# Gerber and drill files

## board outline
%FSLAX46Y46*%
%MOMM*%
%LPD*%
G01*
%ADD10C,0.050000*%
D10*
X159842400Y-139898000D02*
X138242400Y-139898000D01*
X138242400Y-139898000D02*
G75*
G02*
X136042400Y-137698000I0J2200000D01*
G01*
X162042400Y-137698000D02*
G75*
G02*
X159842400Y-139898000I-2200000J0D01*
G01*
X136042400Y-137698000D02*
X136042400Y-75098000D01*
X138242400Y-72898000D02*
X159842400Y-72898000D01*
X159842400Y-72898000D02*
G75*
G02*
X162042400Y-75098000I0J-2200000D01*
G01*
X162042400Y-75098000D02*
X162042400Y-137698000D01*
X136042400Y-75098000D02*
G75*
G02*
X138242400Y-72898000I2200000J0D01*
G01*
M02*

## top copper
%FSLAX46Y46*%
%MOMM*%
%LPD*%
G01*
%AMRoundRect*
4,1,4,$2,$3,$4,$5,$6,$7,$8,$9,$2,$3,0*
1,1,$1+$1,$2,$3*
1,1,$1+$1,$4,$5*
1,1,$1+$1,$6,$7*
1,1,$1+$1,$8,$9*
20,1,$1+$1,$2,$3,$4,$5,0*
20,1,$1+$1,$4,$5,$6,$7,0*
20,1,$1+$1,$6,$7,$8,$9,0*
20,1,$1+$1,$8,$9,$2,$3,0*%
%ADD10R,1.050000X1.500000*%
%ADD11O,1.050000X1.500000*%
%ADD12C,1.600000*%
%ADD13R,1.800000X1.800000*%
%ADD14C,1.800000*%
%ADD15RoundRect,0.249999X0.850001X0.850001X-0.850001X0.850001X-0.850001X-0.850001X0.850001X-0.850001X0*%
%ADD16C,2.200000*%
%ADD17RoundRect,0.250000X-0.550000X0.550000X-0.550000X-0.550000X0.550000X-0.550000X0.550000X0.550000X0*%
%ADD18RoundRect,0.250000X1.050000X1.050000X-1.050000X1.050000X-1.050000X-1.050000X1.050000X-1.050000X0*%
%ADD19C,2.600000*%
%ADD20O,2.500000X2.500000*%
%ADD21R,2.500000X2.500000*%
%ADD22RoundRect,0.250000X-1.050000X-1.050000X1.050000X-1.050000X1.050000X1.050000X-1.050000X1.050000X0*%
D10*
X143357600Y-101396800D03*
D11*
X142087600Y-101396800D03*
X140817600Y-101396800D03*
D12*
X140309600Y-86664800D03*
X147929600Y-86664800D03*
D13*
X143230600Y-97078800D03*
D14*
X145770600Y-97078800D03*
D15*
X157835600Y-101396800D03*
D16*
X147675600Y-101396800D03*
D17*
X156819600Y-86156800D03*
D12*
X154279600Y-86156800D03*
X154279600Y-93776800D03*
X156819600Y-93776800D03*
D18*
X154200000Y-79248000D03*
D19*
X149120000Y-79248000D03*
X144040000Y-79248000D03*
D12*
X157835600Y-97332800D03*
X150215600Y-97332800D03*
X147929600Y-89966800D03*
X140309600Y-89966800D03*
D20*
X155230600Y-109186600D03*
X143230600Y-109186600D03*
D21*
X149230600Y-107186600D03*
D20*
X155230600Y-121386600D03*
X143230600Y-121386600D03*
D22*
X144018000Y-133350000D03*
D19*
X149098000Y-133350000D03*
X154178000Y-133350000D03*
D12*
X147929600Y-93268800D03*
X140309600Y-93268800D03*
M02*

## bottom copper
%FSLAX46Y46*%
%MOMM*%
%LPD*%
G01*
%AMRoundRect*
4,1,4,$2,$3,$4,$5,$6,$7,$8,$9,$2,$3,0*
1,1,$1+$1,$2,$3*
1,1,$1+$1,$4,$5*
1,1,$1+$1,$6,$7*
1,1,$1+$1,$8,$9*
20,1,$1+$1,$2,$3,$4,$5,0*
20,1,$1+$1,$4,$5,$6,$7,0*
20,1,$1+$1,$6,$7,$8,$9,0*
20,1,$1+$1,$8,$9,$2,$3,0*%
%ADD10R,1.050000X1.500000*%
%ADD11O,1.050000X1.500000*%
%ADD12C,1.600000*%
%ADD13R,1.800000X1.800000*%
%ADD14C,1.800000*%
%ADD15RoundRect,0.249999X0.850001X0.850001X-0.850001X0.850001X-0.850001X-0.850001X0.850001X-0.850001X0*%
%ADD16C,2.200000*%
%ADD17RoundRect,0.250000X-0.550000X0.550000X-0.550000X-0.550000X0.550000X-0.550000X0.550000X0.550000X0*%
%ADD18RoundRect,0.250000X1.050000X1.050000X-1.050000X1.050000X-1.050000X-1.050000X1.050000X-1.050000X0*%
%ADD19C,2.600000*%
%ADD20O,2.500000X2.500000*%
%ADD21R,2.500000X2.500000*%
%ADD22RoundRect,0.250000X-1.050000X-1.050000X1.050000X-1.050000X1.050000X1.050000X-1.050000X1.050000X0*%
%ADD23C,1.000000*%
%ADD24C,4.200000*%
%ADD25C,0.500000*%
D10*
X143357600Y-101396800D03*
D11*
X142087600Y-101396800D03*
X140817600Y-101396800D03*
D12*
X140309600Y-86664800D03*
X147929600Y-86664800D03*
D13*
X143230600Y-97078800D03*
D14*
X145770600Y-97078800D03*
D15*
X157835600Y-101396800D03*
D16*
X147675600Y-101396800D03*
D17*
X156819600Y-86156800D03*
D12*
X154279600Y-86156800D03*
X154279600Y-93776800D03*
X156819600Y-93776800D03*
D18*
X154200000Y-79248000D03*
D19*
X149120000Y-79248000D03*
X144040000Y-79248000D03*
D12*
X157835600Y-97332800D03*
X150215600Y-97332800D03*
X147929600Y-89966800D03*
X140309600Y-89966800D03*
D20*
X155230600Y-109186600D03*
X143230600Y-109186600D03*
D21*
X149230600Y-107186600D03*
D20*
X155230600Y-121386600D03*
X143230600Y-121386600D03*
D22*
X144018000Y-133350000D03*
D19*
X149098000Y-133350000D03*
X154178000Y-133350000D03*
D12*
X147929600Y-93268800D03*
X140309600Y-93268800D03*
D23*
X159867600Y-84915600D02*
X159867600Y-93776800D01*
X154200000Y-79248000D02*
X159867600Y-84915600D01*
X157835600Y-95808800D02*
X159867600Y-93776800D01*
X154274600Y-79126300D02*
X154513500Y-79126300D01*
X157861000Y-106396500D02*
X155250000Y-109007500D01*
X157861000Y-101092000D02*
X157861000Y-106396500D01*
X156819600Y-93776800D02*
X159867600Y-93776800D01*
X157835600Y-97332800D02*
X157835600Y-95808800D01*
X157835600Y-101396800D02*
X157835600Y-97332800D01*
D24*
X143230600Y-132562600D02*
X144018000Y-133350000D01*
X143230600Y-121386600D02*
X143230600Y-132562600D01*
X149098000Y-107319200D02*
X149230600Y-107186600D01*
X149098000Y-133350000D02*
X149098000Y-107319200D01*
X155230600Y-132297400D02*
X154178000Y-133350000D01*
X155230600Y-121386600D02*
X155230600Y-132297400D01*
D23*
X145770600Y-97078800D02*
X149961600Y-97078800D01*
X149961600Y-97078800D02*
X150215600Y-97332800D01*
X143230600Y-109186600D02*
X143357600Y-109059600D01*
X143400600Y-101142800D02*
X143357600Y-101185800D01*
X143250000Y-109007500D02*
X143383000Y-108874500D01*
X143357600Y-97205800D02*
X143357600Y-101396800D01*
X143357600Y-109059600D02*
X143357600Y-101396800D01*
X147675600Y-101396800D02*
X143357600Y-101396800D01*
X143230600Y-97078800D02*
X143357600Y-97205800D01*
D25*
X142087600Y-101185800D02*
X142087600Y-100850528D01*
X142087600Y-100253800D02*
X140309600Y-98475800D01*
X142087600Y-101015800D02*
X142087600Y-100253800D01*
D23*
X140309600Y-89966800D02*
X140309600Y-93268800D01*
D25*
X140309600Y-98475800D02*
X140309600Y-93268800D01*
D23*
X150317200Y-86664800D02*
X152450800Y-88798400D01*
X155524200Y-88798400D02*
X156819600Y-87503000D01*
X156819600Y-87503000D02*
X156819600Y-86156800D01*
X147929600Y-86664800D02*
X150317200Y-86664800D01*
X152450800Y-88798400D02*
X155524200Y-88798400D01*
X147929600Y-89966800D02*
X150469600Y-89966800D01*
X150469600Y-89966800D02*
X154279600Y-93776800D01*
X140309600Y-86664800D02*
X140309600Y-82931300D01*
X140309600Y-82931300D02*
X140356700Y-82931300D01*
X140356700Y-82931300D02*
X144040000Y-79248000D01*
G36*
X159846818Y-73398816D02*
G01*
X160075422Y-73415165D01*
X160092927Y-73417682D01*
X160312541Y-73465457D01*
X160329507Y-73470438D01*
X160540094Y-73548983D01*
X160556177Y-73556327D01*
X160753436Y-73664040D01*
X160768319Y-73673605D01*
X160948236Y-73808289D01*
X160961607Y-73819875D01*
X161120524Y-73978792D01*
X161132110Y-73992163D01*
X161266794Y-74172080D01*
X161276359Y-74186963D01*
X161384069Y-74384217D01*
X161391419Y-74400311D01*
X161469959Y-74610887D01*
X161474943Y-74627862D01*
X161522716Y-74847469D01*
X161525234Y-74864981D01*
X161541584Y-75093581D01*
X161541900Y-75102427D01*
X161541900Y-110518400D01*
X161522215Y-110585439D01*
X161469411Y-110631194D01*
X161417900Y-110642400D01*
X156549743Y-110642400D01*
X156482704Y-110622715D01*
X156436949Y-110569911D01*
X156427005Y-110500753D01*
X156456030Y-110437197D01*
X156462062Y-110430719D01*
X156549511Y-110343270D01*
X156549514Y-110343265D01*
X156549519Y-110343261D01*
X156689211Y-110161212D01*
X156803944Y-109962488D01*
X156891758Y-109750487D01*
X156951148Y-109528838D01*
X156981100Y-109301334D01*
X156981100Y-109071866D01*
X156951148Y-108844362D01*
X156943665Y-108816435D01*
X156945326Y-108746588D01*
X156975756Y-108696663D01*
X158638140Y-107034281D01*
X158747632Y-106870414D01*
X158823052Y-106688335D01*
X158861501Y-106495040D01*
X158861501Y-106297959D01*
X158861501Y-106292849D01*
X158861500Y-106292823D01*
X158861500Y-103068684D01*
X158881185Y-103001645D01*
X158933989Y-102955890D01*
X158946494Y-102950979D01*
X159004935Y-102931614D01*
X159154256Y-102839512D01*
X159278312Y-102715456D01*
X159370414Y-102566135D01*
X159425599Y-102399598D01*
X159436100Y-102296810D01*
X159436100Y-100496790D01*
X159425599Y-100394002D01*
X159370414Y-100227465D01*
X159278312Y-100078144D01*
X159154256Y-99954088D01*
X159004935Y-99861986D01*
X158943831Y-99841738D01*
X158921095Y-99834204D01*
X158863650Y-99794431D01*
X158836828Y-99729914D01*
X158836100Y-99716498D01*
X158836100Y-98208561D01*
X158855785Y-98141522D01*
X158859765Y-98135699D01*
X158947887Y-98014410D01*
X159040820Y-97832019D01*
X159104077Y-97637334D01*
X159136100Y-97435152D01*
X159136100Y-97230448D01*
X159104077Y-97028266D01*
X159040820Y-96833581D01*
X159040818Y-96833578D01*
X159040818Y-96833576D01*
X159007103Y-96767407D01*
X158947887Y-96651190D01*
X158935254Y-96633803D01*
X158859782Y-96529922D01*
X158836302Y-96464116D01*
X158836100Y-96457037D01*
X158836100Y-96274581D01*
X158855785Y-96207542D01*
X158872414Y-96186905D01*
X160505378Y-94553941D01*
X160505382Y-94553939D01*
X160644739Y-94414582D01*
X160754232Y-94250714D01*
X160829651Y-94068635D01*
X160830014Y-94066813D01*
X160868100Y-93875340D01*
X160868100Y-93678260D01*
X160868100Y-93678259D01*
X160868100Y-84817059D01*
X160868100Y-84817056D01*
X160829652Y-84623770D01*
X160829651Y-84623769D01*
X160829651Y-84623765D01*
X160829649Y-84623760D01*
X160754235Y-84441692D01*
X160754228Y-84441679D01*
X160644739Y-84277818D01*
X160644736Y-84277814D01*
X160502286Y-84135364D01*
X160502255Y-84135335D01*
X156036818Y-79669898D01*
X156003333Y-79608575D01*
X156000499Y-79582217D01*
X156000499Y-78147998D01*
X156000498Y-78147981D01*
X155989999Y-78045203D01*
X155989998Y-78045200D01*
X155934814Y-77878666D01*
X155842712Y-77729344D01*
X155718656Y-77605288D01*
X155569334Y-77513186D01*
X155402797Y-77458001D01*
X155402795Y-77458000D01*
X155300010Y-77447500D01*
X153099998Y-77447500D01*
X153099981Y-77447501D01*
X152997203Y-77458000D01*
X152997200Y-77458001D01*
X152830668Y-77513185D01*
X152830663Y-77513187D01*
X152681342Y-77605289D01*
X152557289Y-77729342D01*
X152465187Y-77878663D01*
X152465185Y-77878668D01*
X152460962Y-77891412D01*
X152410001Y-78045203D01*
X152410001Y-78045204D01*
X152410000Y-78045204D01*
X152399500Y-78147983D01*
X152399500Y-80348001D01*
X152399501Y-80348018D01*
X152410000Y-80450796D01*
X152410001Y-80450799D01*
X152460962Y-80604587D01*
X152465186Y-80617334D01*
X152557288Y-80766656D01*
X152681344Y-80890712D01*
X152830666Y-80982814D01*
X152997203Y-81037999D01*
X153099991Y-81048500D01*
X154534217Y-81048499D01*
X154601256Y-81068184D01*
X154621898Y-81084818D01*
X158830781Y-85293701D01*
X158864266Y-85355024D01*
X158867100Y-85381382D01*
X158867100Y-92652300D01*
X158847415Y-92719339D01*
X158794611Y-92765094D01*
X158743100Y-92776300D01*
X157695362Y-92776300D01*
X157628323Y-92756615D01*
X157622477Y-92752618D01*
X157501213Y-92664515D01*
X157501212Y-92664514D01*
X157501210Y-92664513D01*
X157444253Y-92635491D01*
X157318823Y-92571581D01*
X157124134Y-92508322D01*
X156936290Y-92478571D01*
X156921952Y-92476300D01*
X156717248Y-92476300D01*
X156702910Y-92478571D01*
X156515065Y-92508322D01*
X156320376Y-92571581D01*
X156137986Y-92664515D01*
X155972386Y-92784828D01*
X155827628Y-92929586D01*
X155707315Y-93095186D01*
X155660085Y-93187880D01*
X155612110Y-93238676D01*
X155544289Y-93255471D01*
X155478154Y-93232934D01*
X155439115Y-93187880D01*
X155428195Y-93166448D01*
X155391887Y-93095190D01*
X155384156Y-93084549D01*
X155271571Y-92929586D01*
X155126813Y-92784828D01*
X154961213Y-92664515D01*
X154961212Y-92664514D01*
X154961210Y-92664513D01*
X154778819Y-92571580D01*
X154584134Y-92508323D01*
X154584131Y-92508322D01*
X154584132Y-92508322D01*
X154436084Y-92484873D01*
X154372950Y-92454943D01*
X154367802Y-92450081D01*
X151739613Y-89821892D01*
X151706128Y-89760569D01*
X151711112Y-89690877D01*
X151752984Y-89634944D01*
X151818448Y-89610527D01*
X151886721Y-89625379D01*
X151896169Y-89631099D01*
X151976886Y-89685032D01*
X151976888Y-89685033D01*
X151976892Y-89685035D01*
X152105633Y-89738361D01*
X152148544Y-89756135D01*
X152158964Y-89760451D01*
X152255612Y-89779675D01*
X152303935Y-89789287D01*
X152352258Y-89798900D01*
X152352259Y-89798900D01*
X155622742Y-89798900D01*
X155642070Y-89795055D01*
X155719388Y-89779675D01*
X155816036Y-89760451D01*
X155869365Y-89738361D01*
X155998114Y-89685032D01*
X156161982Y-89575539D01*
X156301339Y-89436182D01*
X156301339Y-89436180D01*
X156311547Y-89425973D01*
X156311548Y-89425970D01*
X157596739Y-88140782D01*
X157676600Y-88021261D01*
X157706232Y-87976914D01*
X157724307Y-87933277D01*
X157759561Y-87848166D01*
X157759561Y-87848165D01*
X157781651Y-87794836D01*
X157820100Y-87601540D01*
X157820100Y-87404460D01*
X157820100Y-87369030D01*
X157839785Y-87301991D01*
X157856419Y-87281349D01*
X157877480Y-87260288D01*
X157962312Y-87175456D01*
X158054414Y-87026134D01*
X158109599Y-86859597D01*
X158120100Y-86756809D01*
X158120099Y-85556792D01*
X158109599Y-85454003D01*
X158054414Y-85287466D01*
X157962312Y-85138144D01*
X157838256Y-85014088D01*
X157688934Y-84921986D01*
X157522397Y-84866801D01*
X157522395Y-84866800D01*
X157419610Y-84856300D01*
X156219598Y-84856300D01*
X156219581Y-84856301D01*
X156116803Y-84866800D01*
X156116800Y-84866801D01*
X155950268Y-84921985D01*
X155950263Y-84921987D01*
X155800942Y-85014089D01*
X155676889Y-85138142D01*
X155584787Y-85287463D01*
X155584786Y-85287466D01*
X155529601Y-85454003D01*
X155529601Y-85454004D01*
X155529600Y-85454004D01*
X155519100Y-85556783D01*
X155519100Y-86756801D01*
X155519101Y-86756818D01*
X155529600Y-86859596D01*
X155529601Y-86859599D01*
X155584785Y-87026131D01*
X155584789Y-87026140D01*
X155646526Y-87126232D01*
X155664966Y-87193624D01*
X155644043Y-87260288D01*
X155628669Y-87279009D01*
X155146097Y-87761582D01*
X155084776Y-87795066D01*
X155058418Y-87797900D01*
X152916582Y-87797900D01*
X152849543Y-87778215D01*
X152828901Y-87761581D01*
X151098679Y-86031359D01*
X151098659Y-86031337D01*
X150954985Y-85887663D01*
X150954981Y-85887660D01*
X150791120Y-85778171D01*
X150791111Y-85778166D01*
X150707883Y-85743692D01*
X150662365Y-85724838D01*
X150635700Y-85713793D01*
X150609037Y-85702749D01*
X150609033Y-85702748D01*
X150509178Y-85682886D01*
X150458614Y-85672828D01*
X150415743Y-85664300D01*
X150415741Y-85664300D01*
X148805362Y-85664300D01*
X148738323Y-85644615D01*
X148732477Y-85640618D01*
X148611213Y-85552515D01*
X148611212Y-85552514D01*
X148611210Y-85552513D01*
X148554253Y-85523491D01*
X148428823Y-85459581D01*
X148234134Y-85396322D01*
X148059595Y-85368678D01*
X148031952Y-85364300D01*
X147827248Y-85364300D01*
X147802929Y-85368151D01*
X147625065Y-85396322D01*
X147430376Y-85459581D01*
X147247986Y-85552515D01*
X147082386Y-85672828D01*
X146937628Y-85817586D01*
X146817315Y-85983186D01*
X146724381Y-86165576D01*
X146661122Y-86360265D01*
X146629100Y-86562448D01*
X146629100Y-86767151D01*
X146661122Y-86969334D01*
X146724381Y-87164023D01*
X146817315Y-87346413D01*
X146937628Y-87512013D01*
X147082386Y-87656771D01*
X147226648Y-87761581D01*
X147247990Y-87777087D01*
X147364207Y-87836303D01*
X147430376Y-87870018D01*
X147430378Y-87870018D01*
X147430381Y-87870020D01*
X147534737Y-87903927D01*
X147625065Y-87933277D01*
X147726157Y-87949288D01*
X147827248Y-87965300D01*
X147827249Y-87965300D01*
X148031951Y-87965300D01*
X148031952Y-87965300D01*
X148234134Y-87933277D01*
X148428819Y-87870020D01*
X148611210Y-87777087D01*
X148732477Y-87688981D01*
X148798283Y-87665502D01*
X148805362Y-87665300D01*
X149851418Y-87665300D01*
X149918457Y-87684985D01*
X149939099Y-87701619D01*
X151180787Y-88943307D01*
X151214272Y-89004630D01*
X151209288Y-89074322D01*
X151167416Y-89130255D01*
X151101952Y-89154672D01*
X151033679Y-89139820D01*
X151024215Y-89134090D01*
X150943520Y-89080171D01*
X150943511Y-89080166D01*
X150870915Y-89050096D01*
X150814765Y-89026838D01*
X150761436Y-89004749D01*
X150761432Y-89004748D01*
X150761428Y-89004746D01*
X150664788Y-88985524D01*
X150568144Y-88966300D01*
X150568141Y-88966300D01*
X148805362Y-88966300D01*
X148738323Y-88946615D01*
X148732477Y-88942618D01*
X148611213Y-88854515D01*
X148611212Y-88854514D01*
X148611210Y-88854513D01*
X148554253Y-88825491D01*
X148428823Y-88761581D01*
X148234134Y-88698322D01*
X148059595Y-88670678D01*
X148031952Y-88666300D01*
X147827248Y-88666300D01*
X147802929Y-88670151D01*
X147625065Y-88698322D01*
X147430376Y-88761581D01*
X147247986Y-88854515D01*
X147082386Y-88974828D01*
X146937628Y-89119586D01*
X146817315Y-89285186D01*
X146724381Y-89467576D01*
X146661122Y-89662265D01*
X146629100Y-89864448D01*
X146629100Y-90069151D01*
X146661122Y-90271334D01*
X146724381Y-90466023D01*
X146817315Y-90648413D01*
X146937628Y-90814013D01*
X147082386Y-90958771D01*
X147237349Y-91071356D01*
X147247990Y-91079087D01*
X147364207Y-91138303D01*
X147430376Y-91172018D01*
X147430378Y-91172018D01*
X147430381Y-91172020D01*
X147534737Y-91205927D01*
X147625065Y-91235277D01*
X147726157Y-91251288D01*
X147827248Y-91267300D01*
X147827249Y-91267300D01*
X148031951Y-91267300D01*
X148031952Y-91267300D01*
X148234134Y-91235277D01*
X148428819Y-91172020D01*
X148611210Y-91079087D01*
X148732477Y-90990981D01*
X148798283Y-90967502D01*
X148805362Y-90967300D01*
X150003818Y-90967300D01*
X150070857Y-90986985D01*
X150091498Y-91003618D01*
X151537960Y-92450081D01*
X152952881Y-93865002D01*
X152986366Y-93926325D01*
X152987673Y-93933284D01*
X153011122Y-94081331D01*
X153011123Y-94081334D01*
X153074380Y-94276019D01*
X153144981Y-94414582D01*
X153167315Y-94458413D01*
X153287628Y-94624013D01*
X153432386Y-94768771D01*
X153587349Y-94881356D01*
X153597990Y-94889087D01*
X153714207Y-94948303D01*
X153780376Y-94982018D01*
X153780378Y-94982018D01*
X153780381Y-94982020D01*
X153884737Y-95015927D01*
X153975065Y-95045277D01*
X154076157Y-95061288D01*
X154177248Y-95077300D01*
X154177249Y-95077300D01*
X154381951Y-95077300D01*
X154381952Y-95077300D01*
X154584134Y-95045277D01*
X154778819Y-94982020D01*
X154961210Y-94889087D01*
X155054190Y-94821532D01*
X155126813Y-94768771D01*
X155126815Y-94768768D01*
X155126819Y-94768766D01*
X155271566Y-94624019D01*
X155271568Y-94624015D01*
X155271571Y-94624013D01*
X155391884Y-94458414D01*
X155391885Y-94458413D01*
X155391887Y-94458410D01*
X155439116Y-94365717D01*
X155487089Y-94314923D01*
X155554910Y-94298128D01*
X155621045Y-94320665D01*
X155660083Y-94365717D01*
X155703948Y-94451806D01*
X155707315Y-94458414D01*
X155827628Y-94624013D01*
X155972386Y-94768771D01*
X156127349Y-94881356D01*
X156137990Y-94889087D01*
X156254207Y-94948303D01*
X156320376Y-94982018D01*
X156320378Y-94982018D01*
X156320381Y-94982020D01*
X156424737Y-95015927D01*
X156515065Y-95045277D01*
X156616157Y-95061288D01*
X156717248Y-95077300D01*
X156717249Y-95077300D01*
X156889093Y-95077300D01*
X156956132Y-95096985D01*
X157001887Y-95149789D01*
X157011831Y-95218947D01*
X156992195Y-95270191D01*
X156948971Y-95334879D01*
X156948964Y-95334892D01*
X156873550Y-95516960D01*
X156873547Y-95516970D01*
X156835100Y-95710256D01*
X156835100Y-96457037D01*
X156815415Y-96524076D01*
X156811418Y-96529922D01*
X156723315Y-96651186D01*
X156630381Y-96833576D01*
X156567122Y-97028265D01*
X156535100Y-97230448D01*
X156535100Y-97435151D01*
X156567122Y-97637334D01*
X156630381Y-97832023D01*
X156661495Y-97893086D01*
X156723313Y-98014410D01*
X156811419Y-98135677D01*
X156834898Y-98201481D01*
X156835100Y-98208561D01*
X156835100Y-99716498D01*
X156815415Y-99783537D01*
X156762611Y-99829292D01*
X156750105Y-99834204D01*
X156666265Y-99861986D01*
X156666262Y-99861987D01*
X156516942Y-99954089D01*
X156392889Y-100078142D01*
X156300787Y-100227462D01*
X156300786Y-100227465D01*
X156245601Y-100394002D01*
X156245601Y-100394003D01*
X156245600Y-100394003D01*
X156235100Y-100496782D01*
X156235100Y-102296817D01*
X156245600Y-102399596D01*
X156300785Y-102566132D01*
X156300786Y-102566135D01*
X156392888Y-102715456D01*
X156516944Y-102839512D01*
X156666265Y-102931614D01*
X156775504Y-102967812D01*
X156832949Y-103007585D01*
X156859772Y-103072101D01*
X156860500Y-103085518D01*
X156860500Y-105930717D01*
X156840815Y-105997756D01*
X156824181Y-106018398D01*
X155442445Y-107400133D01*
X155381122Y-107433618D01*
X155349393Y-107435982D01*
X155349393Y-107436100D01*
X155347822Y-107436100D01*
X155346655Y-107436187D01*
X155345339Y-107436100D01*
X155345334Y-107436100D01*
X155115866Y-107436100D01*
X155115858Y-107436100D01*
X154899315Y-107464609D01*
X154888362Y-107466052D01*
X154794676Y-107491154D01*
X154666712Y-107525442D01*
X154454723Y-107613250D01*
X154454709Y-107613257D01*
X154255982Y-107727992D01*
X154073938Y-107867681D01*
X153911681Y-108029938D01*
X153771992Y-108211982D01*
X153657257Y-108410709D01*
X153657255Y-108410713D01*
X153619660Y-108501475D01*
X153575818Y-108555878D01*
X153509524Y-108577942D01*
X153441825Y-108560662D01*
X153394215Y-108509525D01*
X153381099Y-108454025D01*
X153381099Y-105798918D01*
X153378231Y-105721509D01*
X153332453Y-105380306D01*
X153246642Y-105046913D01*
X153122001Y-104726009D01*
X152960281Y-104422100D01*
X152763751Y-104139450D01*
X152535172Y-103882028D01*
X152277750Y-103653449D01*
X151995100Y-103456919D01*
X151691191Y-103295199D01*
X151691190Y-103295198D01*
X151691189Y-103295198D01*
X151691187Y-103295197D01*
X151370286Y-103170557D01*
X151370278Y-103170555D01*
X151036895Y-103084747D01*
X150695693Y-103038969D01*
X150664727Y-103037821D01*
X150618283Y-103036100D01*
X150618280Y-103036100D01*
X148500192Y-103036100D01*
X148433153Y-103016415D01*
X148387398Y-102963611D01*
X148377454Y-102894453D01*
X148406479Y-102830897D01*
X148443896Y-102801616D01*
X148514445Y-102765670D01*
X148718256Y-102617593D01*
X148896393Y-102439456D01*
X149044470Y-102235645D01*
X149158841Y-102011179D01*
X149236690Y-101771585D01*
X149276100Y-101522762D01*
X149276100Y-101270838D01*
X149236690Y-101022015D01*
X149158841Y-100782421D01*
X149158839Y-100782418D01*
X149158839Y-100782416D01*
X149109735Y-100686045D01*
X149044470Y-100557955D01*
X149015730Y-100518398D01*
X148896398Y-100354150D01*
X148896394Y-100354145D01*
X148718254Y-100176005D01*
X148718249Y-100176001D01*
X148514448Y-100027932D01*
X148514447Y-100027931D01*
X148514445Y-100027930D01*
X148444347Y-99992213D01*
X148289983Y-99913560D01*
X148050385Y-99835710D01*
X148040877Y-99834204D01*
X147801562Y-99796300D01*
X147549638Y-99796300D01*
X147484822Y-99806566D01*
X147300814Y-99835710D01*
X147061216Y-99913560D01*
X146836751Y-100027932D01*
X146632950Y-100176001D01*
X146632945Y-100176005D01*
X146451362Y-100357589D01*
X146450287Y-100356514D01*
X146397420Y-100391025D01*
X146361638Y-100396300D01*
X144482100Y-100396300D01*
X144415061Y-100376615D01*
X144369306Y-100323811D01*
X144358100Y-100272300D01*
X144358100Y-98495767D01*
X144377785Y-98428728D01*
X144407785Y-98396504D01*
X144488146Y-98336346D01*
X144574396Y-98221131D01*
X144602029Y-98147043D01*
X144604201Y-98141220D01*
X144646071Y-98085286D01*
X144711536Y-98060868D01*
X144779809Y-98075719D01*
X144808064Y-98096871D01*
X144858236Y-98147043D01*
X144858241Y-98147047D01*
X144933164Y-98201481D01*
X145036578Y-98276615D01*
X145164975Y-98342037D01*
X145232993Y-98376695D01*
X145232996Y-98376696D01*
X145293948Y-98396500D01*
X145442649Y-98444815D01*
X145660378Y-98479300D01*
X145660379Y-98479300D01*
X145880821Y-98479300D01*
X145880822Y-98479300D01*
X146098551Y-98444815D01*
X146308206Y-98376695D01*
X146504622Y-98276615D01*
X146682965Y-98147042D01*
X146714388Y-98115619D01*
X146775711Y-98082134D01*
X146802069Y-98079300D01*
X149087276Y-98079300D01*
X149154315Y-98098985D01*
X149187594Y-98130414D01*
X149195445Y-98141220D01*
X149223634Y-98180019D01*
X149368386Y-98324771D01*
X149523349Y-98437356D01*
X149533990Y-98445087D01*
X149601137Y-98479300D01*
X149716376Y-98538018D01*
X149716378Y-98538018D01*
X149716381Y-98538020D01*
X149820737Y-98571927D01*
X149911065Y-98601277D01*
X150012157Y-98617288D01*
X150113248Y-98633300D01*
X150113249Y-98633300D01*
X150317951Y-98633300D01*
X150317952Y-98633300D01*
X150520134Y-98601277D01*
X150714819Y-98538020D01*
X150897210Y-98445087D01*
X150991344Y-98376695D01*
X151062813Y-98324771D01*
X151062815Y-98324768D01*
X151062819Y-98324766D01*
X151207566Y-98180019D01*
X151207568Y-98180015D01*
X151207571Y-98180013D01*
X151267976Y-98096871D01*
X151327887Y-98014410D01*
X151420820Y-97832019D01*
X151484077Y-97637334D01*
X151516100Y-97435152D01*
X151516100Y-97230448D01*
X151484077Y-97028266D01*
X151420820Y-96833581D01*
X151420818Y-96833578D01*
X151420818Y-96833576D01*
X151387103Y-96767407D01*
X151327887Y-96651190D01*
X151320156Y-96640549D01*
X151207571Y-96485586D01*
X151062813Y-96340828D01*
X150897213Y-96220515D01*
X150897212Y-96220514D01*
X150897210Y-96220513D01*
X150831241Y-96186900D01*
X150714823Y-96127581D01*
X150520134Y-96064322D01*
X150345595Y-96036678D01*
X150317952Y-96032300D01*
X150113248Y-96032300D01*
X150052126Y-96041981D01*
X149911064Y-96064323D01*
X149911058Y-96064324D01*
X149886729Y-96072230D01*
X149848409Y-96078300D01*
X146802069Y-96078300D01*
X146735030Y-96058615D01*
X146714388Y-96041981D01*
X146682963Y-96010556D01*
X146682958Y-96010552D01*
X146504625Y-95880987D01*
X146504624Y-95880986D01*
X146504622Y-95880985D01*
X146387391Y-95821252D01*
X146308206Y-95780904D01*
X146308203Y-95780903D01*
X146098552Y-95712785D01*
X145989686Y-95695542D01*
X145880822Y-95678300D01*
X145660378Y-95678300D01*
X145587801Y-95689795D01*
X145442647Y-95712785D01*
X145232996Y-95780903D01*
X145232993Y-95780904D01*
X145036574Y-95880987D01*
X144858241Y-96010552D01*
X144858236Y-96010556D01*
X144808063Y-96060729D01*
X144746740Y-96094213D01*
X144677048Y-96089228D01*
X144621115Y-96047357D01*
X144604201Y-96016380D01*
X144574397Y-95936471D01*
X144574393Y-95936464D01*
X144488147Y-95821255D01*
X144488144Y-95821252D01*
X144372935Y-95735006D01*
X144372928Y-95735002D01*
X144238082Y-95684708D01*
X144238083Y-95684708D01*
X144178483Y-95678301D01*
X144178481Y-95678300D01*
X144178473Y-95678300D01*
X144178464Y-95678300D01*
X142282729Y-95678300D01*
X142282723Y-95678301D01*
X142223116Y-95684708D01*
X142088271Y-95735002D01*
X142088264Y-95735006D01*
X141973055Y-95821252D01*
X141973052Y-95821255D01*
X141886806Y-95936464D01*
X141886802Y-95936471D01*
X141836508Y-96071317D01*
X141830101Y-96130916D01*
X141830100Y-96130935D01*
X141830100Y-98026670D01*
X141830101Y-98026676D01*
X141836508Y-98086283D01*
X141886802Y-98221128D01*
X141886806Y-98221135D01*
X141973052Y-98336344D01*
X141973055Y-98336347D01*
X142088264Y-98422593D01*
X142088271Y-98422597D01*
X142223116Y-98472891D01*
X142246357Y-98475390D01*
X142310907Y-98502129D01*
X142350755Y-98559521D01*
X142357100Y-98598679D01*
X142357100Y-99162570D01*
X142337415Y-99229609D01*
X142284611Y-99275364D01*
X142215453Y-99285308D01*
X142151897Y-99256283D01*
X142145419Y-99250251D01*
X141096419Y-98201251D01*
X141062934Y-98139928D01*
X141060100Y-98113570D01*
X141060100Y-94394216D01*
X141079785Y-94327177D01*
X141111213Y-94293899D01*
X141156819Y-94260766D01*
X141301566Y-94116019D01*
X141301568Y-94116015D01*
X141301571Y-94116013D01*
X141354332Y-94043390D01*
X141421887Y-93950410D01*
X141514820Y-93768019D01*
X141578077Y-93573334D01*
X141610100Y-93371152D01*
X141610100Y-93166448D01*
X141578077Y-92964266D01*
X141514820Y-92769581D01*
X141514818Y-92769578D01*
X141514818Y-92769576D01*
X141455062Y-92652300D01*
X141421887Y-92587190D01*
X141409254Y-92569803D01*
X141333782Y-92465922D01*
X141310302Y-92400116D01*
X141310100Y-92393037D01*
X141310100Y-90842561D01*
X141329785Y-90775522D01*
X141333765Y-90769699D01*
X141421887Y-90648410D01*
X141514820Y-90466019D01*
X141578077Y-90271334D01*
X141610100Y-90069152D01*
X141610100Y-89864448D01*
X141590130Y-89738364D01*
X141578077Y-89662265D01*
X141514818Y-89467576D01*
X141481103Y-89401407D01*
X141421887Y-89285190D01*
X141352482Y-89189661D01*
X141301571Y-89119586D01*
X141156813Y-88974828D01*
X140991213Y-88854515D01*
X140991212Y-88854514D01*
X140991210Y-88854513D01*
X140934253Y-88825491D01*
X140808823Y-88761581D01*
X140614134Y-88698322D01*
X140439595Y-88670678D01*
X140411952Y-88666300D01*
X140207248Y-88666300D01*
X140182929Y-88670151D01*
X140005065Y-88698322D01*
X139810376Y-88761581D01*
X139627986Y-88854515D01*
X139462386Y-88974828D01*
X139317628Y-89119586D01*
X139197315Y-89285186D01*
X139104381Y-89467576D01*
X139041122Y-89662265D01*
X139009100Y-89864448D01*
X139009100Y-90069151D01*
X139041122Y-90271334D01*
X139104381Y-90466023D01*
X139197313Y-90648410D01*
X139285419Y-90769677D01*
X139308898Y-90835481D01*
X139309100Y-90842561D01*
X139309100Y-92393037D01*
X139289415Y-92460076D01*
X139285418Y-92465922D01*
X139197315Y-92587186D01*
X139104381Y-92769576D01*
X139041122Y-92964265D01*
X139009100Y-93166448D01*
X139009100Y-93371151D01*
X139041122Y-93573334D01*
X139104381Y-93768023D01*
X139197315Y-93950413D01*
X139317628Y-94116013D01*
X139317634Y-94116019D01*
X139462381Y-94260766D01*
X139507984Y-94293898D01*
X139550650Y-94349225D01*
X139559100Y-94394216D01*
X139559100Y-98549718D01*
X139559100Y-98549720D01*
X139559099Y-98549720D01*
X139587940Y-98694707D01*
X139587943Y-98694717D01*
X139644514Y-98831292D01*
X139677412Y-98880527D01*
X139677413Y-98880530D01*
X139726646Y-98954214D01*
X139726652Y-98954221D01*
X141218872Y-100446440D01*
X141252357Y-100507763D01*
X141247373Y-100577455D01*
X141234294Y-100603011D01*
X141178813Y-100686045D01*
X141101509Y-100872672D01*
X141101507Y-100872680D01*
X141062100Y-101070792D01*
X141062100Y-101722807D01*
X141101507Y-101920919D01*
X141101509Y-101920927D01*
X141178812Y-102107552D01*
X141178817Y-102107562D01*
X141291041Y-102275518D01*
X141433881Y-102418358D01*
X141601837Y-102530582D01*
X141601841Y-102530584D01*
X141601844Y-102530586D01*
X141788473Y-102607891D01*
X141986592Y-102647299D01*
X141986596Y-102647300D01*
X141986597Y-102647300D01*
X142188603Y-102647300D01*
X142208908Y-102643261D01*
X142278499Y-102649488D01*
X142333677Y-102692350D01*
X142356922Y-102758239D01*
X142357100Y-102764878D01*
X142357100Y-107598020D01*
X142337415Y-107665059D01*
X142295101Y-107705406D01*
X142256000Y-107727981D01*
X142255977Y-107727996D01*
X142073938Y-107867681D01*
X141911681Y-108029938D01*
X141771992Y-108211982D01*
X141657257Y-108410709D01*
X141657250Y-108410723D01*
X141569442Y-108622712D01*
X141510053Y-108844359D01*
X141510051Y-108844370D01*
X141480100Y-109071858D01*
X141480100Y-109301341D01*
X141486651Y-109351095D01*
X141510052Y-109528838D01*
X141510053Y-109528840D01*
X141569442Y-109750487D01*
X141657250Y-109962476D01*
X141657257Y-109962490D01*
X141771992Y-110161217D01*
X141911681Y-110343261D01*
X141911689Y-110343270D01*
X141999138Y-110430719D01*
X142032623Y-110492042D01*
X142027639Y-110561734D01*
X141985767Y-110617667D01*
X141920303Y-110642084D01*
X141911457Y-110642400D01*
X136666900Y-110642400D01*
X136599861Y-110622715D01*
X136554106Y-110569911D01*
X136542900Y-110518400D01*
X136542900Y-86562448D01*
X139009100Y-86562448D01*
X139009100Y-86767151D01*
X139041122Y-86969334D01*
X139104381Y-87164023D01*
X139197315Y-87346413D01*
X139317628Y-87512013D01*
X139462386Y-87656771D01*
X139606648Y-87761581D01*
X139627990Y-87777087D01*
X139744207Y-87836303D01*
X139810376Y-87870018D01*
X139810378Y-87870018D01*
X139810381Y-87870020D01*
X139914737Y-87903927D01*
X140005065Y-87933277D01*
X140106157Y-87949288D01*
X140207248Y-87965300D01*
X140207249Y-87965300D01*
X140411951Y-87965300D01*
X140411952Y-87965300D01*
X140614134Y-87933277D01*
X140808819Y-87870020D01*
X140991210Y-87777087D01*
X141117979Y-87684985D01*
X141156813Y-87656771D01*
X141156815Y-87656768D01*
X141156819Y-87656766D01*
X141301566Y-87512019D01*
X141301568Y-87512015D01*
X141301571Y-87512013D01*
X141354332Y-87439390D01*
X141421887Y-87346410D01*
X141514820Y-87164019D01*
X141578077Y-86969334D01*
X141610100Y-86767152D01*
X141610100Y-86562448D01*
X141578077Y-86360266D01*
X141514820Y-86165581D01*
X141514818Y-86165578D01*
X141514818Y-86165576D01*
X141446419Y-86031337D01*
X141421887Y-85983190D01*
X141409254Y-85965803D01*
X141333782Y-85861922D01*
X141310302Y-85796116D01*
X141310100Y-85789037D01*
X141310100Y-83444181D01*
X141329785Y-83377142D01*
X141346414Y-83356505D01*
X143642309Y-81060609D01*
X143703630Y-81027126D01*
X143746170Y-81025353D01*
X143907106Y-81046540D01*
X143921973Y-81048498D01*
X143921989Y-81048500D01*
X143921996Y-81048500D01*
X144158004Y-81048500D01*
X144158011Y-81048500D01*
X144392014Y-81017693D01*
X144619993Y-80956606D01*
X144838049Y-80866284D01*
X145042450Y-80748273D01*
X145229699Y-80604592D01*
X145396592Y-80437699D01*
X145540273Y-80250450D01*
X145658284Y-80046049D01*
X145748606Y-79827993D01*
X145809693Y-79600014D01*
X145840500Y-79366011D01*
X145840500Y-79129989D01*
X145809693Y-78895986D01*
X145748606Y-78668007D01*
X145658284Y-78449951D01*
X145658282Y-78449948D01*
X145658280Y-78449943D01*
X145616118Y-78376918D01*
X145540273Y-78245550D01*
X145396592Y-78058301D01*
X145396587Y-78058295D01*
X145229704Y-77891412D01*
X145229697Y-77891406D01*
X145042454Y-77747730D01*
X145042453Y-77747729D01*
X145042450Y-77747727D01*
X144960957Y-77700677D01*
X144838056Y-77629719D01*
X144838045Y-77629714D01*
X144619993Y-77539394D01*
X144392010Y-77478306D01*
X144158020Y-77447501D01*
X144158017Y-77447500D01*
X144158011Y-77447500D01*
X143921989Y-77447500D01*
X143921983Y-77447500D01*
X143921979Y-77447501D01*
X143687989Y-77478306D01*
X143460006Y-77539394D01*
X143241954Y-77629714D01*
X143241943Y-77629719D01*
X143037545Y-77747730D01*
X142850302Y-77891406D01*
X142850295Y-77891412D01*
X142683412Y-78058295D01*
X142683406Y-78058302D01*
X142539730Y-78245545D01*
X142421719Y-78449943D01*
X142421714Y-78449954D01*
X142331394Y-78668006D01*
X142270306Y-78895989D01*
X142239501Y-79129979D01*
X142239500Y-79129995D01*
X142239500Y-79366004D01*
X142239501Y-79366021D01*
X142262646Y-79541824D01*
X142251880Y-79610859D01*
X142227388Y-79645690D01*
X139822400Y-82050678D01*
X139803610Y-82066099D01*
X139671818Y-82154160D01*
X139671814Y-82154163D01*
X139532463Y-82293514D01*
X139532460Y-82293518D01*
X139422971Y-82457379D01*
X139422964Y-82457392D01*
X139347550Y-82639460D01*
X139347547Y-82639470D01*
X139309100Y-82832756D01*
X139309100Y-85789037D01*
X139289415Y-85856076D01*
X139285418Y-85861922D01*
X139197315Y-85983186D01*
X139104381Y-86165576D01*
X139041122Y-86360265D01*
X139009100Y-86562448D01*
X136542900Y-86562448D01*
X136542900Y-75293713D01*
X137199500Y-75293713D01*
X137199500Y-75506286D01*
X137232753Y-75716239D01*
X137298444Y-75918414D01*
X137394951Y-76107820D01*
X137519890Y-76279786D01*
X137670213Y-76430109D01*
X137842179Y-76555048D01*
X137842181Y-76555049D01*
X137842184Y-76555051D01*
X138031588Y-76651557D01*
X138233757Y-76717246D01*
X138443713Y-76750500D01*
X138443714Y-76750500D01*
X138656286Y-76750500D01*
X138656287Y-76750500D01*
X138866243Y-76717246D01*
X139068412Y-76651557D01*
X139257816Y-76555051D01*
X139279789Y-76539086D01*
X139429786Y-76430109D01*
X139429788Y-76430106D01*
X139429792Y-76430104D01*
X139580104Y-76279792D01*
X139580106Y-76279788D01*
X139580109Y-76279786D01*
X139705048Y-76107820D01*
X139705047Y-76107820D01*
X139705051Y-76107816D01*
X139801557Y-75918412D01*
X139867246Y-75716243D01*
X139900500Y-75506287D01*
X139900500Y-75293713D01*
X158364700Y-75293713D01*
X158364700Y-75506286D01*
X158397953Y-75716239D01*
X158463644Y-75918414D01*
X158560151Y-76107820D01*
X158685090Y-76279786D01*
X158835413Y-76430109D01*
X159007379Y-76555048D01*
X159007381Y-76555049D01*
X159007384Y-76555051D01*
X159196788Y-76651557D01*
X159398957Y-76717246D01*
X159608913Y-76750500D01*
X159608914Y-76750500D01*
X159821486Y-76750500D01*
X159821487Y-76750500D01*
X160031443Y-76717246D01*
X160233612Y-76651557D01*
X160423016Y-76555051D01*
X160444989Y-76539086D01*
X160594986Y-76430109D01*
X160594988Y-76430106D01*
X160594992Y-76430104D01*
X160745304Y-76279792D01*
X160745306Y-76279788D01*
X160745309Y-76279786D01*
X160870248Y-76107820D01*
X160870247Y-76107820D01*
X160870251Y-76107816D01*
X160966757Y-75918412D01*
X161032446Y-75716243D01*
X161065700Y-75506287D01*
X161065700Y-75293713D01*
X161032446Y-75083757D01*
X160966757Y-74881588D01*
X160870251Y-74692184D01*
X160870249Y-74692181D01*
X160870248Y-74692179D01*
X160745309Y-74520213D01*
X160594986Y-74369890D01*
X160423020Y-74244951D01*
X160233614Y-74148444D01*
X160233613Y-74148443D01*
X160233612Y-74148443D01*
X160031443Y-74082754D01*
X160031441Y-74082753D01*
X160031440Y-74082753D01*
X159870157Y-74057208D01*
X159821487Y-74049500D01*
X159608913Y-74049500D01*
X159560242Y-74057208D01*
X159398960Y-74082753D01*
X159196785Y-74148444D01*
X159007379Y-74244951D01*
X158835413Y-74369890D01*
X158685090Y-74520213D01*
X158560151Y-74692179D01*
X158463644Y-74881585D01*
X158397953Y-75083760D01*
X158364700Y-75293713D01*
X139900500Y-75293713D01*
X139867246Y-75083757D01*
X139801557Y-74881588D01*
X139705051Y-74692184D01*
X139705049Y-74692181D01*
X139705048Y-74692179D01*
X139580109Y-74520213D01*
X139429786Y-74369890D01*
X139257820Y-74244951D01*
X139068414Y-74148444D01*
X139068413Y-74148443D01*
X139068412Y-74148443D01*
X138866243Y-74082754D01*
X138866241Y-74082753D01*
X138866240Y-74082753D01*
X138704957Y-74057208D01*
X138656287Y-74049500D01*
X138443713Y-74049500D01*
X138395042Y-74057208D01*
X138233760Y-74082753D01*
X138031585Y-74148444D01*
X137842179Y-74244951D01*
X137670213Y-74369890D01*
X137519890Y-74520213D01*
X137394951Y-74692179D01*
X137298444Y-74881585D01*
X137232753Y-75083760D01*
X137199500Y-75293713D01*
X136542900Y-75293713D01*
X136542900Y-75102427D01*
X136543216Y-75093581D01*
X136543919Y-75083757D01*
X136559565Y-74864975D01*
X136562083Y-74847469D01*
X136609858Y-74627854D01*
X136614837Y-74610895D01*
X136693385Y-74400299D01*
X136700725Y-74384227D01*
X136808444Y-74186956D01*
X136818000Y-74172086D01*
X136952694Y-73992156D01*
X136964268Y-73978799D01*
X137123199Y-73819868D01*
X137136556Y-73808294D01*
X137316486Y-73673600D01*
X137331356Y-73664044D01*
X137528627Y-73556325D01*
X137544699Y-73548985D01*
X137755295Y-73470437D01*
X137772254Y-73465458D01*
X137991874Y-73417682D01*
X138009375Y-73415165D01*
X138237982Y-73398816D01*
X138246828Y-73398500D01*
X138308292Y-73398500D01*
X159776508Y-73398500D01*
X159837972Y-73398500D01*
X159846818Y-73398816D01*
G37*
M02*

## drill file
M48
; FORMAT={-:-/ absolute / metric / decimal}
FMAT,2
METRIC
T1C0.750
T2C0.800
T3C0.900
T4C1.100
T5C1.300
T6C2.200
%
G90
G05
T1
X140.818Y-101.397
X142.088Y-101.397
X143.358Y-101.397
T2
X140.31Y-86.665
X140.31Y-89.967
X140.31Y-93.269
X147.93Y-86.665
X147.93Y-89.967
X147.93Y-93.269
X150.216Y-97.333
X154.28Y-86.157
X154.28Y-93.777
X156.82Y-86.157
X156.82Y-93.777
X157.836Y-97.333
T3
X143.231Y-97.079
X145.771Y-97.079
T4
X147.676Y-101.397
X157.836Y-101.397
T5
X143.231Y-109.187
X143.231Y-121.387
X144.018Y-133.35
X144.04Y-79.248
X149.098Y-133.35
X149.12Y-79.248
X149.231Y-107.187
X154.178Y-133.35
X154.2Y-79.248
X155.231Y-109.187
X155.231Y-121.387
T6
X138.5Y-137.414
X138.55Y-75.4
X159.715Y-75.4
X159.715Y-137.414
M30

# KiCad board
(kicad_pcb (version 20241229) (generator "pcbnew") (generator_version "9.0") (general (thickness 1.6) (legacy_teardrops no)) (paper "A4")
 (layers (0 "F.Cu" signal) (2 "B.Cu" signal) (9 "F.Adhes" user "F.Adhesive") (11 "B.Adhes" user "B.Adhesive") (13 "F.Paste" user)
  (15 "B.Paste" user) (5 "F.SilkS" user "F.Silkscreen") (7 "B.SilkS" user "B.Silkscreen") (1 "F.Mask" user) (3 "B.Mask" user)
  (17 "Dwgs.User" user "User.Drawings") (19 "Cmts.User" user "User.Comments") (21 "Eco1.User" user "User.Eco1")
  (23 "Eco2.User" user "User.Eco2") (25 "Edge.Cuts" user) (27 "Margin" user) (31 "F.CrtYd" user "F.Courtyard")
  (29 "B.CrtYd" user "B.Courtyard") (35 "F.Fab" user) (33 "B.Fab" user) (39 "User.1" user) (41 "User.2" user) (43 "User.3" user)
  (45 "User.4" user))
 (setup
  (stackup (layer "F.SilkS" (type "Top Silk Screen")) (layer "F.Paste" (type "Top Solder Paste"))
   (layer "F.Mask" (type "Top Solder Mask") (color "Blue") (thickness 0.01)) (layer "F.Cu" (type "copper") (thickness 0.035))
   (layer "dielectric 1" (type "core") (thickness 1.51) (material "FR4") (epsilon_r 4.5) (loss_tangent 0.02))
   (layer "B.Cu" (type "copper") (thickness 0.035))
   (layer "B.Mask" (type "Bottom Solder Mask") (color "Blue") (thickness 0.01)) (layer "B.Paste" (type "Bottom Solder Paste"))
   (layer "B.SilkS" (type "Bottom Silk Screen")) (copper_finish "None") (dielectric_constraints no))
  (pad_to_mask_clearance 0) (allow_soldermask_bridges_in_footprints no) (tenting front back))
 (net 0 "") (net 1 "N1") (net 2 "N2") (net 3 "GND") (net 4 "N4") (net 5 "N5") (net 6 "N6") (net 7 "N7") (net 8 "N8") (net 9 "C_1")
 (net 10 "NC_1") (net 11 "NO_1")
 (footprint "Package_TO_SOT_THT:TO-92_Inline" (layer "F.Cu") (at 143.3576 101.3968 180)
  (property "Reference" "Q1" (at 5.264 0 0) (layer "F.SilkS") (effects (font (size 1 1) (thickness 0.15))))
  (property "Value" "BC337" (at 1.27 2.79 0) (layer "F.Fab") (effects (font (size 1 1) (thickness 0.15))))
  (pad "1" thru_hole rect (at 0 0 180) (size 1.05 1.5) (drill 0.75) (layers "*.Cu" "*.Mask") (remove_unused_layers no) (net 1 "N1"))
  (pad "2" thru_hole oval (at 1.27 0 180) (size 1.05 1.5) (drill 0.75) (layers "*.Cu" "*.Mask") (remove_unused_layers no) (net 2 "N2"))
  (pad "3" thru_hole oval (at 2.54 0 180) (size 1.05 1.5) (drill 0.75) (layers "*.Cu" "*.Mask") (remove_unused_layers no) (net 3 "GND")))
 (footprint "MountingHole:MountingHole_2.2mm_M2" (layer "F.Cu") (at 159.7152 137.414)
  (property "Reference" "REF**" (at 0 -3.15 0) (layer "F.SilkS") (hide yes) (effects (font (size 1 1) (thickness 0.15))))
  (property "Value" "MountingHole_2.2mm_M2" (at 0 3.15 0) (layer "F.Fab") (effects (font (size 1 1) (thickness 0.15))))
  (pad "" np_thru_hole circle (at 0 0) (size 2.2 2.2) (drill 2.2) (layers "*.Cu" "*.Mask")))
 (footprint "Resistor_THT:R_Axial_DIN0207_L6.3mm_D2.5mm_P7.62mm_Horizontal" (layer "F.Cu") (at 140.3096 86.6648)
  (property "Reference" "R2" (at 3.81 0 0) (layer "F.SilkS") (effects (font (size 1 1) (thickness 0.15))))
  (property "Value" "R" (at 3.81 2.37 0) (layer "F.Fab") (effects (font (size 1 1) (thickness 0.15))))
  (pad "1" thru_hole circle (at 0 0) (size 1.6 1.6) (drill 0.8) (layers "*.Cu" "*.Mask") (remove_unused_layers no) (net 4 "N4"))
  (pad "2" thru_hole circle (at 7.62 0) (size 1.6 1.6) (drill 0.8) (layers "*.Cu" "*.Mask") (remove_unused_layers no) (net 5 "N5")))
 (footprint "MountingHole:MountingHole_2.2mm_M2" (layer "F.Cu") (at 159.7152 75.4)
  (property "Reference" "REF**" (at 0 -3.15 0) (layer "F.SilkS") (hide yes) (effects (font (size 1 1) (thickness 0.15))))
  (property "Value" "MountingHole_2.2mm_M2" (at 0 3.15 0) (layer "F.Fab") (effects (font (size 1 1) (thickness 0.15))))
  (pad "" np_thru_hole circle (at 0 0) (size 2.2 2.2) (drill 2.2) (layers "*.Cu" "*.Mask")))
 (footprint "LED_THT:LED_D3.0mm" (layer "F.Cu") (at 143.2306 97.0788)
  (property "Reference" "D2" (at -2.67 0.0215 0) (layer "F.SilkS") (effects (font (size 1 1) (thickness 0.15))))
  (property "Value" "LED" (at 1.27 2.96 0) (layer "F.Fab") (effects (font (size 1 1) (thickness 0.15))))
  (pad "1" thru_hole rect (at 0 0) (size 1.8 1.8) (drill 0.9) (layers "*.Cu" "*.Mask") (remove_unused_layers no) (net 1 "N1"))
  (pad "2" thru_hole circle (at 2.54 0) (size 1.8 1.8) (drill 0.9) (layers "*.Cu" "*.Mask") (remove_unused_layers no) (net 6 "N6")))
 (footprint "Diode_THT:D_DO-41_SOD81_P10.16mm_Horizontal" (layer "F.Cu") (at 157.8356 101.3968 180)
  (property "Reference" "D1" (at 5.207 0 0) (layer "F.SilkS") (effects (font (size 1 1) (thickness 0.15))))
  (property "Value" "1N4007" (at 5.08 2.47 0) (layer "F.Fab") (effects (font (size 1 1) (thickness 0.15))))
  (pad "1" thru_hole roundrect (at 0 0 180) (size 2.2 2.2) (drill 1.1) (layers "*.Cu" "*.Mask") (remove_unused_layers no)
   (roundrect_rratio 0.113636) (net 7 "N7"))
  (pad "2" thru_hole circle (at 10.16 0 180) (size 2.2 2.2) (drill 1.1) (layers "*.Cu" "*.Mask") (remove_unused_layers no) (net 1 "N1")))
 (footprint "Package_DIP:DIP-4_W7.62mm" (layer "F.Cu") (at 156.8196 86.1568 -90)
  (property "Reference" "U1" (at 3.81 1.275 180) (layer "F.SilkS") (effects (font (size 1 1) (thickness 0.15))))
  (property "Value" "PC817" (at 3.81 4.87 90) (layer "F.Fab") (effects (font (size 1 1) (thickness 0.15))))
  (pad "1" thru_hole roundrect (at 0 0 270) (size 1.6 1.6) (drill 0.8) (layers "*.Cu" "*.Mask") (remove_unused_layers no)
   (roundrect_rratio 0.15625) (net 5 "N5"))
  (pad "2" thru_hole circle (at 0 2.54 270) (size 1.6 1.6) (drill 0.8) (layers "*.Cu" "*.Mask") (remove_unused_layers no) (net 3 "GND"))
  (pad "3" thru_hole circle (at 7.62 2.54 270) (size 1.6 1.6) (drill 0.8) (layers "*.Cu" "*.Mask") (remove_unused_layers no) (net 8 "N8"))
  (pad "4" thru_hole circle (at 7.62 0 270) (size 1.6 1.6) (drill 0.8) (layers "*.Cu" "*.Mask") (remove_unused_layers no) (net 7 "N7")))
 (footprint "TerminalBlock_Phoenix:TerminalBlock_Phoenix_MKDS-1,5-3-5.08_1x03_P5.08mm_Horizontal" (layer "F.Cu") (at 154.2 79.248 180)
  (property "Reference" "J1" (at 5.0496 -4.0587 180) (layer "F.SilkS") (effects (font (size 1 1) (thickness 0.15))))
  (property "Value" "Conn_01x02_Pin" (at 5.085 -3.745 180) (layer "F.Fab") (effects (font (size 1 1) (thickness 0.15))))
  (pad "1" thru_hole roundrect (at 0 0 180) (size 2.6 2.6) (drill 1.3) (layers "*.Cu" "*.Mask") (remove_unused_layers no)
   (roundrect_rratio 0.096154) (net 7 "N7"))
  (pad "2" thru_hole circle (at 5.08 0 180) (size 2.6 2.6) (drill 1.3) (layers "*.Cu" "*.Mask") (remove_unused_layers no) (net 3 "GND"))
  (pad "3" thru_hole circle (at 10.16 0 180) (size 2.6 2.6) (drill 1.3) (layers "*.Cu" "*.Mask") (remove_unused_layers no) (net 4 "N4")))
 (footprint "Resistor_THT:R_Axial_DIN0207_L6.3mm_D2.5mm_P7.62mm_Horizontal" (layer "F.Cu") (at 157.8356 97.3328 180)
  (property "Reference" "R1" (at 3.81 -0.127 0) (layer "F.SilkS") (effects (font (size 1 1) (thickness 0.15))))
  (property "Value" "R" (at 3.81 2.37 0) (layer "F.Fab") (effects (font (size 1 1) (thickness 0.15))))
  (pad "1" thru_hole circle (at 0 0 180) (size 1.6 1.6) (drill 0.8) (layers "*.Cu" "*.Mask") (remove_unused_layers no) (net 7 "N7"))
  (pad "2" thru_hole circle (at 7.62 0 180) (size 1.6 1.6) (drill 0.8) (layers "*.Cu" "*.Mask") (remove_unused_layers no) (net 6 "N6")))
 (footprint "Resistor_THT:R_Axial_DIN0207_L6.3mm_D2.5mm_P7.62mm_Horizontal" (layer "F.Cu") (at 147.9296 89.9668 180)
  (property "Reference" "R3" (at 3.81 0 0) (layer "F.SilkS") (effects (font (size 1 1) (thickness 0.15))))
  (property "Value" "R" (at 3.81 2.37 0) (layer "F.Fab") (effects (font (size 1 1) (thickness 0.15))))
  (pad "1" thru_hole circle (at 0 0 180) (size 1.6 1.6) (drill 0.8) (layers "*.Cu" "*.Mask") (remove_unused_layers no) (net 8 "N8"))
  (pad "2" thru_hole circle (at 7.62 0 180) (size 1.6 1.6) (drill 0.8) (layers "*.Cu" "*.Mask") (remove_unused_layers no) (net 2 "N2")))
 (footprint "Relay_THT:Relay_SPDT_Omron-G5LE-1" (layer "F.Cu") (at 149.2306 107.1866)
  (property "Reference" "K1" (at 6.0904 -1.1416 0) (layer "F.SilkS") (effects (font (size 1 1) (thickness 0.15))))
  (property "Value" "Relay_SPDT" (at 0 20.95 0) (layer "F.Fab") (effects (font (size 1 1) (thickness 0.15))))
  (pad "1" thru_hole oval (at 6 2) (size 2.5 2.5) (drill 1.3) (layers "*.Cu" "*.Mask") (remove_unused_layers no) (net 7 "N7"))
  (pad "2" thru_hole oval (at -6 2) (size 2.5 2.5) (drill 1.3) (layers "*.Cu" "*.Mask") (remove_unused_layers no) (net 1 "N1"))
  (pad "3" thru_hole rect (at 0 0) (size 2.5 2.5) (drill 1.3) (layers "*.Cu" "*.Mask") (remove_unused_layers no) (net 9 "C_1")
   (clearance 2.9))
  (pad "4" thru_hole oval (at 6 14.2) (size 2.5 2.5) (drill 1.3) (layers "*.Cu" "*.Mask") (remove_unused_layers no) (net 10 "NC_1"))
  (pad "5" thru_hole oval (at -6 14.2) (size 2.5 2.5) (drill 1.3) (layers "*.Cu" "*.Mask") (remove_unused_layers no) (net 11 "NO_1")))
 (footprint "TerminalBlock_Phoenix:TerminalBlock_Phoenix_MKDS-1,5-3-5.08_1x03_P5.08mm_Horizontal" (layer "F.Cu") (at 144.018 133.35)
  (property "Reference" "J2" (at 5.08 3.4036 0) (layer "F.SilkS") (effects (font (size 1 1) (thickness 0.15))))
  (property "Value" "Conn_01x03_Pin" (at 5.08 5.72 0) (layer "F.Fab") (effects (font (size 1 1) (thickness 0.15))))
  (pad "1" thru_hole roundrect (at 0 0) (size 2.6 2.6) (drill 1.3) (layers "*.Cu" "*.Mask") (remove_unused_layers no)
   (roundrect_rratio 0.096154) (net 11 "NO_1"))
  (pad "2" thru_hole circle (at 5.08 0) (size 2.6 2.6) (drill 1.3) (layers "*.Cu" "*.Mask") (remove_unused_layers no) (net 9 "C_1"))
  (pad "3" thru_hole circle (at 10.16 0) (size 2.6 2.6) (drill 1.3) (layers "*.Cu" "*.Mask") (remove_unused_layers no) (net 10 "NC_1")))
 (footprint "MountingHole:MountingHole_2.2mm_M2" (layer "F.Cu") (at 138.5 137.414)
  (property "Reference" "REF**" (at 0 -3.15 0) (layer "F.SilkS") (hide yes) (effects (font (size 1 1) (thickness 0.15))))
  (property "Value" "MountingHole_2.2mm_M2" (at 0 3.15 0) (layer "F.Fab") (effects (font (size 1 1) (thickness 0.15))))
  (pad "" np_thru_hole circle (at 0 0) (size 2.2 2.2) (drill 2.2) (layers "*.Cu" "*.Mask")))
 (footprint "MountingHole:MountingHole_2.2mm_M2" (layer "F.Cu") (at 138.55 75.4)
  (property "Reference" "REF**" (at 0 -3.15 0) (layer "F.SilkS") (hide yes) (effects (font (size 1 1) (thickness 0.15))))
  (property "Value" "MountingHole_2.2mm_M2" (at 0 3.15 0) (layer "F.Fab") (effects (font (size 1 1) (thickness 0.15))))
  (pad "" np_thru_hole circle (at 0 0) (size 2.2 2.2) (drill 2.2) (layers "*.Cu" "*.Mask")))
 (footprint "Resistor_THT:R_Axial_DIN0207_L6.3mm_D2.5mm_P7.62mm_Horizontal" (layer "F.Cu") (at 147.9296 93.2688 180)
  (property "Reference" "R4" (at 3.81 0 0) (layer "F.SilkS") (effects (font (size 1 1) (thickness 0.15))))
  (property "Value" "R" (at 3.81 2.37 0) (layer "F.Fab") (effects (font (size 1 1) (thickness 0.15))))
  (pad "1" thru_hole circle (at 0 0 180) (size 1.6 1.6) (drill 0.8) (layers "*.Cu" "*.Mask") (remove_unused_layers no) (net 3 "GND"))
  (pad "2" thru_hole circle (at 7.62 0 180) (size 1.6 1.6) (drill 0.8) (layers "*.Cu" "*.Mask") (remove_unused_layers no) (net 2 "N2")))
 (gr_line (start 159.8424 139.898) (end 138.2424 139.898) (stroke (width 0.05) (type default)) (layer "Edge.Cuts"))
 (gr_arc (start 138.2424 139.898) (mid 136.686765 139.253635) (end 136.0424 137.698) (stroke (width 0.05) (type default))
  (layer "Edge.Cuts"))
 (gr_arc (start 162.0424 137.698) (mid 161.398035 139.253635) (end 159.8424 139.898) (stroke (width 0.05) (type default))
  (layer "Edge.Cuts"))
 (gr_line (start 136.0424 137.698) (end 136.0424 75.098) (stroke (width 0.05) (type default)) (layer "Edge.Cuts"))
 (gr_line (start 138.2424 72.898) (end 159.8424 72.898) (stroke (width 0.05) (type default)) (layer "Edge.Cuts"))
 (gr_arc (start 159.8424 72.898) (mid 161.398035 73.542365) (end 162.0424 75.098) (stroke (width 0.05) (type default)) (layer "Edge.Cuts"))
 (gr_line (start 162.0424 75.098) (end 162.0424 137.698) (stroke (width 0.05) (type default)) (layer "Edge.Cuts"))
 (gr_arc (start 136.0424 75.098) (mid 136.686765 73.542365) (end 138.2424 72.898) (stroke (width 0.05) (type default)) (layer "Edge.Cuts"))
 (segment (start 159.8676 84.9156) (end 159.8676 93.7768) (width 1) (layer "B.Cu") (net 7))
 (segment (start 154.2 79.248) (end 159.8676 84.9156) (width 1) (layer "B.Cu") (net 7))
 (segment (start 157.8356 95.8088) (end 159.8676 93.7768) (width 1) (layer "B.Cu") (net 7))
 (segment (start 154.2746 79.1263) (end 154.5135 79.1263) (width 1) (layer "B.Cu") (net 7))
 (segment (start 157.861 106.3965) (end 155.25 109.0075) (width 1) (layer "B.Cu") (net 7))
 (segment (start 157.861 101.092) (end 157.861 106.3965) (width 1) (layer "B.Cu") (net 7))
 (segment (start 156.8196 93.7768) (end 159.8676 93.7768) (width 1) (layer "B.Cu") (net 7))
 (segment (start 157.8356 97.3328) (end 157.8356 95.8088) (width 1) (layer "B.Cu") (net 7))
 (segment (start 157.8356 101.3968) (end 157.8356 97.3328) (width 1) (layer "B.Cu") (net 7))
 (segment (start 143.2306 132.5626) (end 144.018 133.35) (width 4.2) (layer "B.Cu") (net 11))
 (segment (start 143.2306 121.3866) (end 143.2306 132.5626) (width 4.2) (layer "B.Cu") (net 11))
 (segment (start 149.098 107.3192) (end 149.2306 107.1866) (width 4.2) (layer "B.Cu") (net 9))
 (segment (start 149.098 133.35) (end 149.098 107.3192) (width 4.2) (layer "B.Cu") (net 9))
 (segment (start 155.2306 132.2974) (end 154.178 133.35) (width 4.2) (layer "B.Cu") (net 10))
 (segment (start 155.2306 121.3866) (end 155.2306 132.2974) (width 4.2) (layer "B.Cu") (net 10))
 (segment (start 145.7706 97.0788) (end 149.9616 97.0788) (width 1) (layer "B.Cu") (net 6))
 (segment (start 149.9616 97.0788) (end 150.2156 97.3328) (width 1) (layer "B.Cu") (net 6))
 (segment (start 143.2306 109.1866) (end 143.3576 109.0596) (width 1) (layer "B.Cu") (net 1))
 (segment (start 143.4006 101.1428) (end 143.3576 101.1858) (width 1) (layer "B.Cu") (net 1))
 (segment (start 143.25 109.0075) (end 143.383 108.8745) (width 1) (layer "B.Cu") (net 1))
 (segment (start 143.3576 97.2058) (end 143.3576 101.3968) (width 1) (layer "B.Cu") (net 1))
 (segment (start 143.3576 109.0596) (end 143.3576 101.3968) (width 1) (layer "B.Cu") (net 1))
 (segment (start 147.6756 101.3968) (end 143.3576 101.3968) (width 1) (layer "B.Cu") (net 1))
 (segment (start 143.2306 97.0788) (end 143.3576 97.2058) (width 1) (layer "B.Cu") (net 1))
 (segment (start 142.0876 101.1858) (end 142.0876 100.850528) (width 0.5) (layer "B.Cu") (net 2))
 (segment (start 142.0876 100.2538) (end 140.3096 98.4758) (width 0.5) (layer "B.Cu") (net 2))
 (segment (start 142.0876 101.0158) (end 142.0876 100.2538) (width 0.5) (layer "B.Cu") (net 2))
 (segment (start 140.3096 89.9668) (end 140.3096 93.2688) (width 1) (layer "B.Cu") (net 2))
 (segment (start 140.3096 98.4758) (end 140.3096 93.2688) (width 0.5) (layer "B.Cu") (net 2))
 (segment (start 150.3172 86.6648) (end 152.4508 88.7984) (width 1) (layer "B.Cu") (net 5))
 (segment (start 155.5242 88.7984) (end 156.8196 87.503) (width 1) (layer "B.Cu") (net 5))
 (segment (start 156.8196 87.503) (end 156.8196 86.1568) (width 1) (layer "B.Cu") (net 5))
 (segment (start 147.9296 86.6648) (end 150.3172 86.6648) (width 1) (layer "B.Cu") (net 5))
 (segment (start 152.4508 88.7984) (end 155.5242 88.7984) (width 1) (layer "B.Cu") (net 5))
 (segment (start 147.9296 89.9668) (end 150.4696 89.9668) (width 1) (layer "B.Cu") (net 8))
 (segment (start 150.4696 89.9668) (end 154.2796 93.7768) (width 1) (layer "B.Cu") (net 8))
 (segment (start 140.3096 86.6648) (end 140.3096 82.9313) (width 1) (layer "B.Cu") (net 4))
 (segment (start 140.3096 82.9313) (end 140.3567 82.9313) (width 1) (layer "B.Cu") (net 4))
 (segment (start 140.3567 82.9313) (end 144.04 79.248) (width 1) (layer "B.Cu") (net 4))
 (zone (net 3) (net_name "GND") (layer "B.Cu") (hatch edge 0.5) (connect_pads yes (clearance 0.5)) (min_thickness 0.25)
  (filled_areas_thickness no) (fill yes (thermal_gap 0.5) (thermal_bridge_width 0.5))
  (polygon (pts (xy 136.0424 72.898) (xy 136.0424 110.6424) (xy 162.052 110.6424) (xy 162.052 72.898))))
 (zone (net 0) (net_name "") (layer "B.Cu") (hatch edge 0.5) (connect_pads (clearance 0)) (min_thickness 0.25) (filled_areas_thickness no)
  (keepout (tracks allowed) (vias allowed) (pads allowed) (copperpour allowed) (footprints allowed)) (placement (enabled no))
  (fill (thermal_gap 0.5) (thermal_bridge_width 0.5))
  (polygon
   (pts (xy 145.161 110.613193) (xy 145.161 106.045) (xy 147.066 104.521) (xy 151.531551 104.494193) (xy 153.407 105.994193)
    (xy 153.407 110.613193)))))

